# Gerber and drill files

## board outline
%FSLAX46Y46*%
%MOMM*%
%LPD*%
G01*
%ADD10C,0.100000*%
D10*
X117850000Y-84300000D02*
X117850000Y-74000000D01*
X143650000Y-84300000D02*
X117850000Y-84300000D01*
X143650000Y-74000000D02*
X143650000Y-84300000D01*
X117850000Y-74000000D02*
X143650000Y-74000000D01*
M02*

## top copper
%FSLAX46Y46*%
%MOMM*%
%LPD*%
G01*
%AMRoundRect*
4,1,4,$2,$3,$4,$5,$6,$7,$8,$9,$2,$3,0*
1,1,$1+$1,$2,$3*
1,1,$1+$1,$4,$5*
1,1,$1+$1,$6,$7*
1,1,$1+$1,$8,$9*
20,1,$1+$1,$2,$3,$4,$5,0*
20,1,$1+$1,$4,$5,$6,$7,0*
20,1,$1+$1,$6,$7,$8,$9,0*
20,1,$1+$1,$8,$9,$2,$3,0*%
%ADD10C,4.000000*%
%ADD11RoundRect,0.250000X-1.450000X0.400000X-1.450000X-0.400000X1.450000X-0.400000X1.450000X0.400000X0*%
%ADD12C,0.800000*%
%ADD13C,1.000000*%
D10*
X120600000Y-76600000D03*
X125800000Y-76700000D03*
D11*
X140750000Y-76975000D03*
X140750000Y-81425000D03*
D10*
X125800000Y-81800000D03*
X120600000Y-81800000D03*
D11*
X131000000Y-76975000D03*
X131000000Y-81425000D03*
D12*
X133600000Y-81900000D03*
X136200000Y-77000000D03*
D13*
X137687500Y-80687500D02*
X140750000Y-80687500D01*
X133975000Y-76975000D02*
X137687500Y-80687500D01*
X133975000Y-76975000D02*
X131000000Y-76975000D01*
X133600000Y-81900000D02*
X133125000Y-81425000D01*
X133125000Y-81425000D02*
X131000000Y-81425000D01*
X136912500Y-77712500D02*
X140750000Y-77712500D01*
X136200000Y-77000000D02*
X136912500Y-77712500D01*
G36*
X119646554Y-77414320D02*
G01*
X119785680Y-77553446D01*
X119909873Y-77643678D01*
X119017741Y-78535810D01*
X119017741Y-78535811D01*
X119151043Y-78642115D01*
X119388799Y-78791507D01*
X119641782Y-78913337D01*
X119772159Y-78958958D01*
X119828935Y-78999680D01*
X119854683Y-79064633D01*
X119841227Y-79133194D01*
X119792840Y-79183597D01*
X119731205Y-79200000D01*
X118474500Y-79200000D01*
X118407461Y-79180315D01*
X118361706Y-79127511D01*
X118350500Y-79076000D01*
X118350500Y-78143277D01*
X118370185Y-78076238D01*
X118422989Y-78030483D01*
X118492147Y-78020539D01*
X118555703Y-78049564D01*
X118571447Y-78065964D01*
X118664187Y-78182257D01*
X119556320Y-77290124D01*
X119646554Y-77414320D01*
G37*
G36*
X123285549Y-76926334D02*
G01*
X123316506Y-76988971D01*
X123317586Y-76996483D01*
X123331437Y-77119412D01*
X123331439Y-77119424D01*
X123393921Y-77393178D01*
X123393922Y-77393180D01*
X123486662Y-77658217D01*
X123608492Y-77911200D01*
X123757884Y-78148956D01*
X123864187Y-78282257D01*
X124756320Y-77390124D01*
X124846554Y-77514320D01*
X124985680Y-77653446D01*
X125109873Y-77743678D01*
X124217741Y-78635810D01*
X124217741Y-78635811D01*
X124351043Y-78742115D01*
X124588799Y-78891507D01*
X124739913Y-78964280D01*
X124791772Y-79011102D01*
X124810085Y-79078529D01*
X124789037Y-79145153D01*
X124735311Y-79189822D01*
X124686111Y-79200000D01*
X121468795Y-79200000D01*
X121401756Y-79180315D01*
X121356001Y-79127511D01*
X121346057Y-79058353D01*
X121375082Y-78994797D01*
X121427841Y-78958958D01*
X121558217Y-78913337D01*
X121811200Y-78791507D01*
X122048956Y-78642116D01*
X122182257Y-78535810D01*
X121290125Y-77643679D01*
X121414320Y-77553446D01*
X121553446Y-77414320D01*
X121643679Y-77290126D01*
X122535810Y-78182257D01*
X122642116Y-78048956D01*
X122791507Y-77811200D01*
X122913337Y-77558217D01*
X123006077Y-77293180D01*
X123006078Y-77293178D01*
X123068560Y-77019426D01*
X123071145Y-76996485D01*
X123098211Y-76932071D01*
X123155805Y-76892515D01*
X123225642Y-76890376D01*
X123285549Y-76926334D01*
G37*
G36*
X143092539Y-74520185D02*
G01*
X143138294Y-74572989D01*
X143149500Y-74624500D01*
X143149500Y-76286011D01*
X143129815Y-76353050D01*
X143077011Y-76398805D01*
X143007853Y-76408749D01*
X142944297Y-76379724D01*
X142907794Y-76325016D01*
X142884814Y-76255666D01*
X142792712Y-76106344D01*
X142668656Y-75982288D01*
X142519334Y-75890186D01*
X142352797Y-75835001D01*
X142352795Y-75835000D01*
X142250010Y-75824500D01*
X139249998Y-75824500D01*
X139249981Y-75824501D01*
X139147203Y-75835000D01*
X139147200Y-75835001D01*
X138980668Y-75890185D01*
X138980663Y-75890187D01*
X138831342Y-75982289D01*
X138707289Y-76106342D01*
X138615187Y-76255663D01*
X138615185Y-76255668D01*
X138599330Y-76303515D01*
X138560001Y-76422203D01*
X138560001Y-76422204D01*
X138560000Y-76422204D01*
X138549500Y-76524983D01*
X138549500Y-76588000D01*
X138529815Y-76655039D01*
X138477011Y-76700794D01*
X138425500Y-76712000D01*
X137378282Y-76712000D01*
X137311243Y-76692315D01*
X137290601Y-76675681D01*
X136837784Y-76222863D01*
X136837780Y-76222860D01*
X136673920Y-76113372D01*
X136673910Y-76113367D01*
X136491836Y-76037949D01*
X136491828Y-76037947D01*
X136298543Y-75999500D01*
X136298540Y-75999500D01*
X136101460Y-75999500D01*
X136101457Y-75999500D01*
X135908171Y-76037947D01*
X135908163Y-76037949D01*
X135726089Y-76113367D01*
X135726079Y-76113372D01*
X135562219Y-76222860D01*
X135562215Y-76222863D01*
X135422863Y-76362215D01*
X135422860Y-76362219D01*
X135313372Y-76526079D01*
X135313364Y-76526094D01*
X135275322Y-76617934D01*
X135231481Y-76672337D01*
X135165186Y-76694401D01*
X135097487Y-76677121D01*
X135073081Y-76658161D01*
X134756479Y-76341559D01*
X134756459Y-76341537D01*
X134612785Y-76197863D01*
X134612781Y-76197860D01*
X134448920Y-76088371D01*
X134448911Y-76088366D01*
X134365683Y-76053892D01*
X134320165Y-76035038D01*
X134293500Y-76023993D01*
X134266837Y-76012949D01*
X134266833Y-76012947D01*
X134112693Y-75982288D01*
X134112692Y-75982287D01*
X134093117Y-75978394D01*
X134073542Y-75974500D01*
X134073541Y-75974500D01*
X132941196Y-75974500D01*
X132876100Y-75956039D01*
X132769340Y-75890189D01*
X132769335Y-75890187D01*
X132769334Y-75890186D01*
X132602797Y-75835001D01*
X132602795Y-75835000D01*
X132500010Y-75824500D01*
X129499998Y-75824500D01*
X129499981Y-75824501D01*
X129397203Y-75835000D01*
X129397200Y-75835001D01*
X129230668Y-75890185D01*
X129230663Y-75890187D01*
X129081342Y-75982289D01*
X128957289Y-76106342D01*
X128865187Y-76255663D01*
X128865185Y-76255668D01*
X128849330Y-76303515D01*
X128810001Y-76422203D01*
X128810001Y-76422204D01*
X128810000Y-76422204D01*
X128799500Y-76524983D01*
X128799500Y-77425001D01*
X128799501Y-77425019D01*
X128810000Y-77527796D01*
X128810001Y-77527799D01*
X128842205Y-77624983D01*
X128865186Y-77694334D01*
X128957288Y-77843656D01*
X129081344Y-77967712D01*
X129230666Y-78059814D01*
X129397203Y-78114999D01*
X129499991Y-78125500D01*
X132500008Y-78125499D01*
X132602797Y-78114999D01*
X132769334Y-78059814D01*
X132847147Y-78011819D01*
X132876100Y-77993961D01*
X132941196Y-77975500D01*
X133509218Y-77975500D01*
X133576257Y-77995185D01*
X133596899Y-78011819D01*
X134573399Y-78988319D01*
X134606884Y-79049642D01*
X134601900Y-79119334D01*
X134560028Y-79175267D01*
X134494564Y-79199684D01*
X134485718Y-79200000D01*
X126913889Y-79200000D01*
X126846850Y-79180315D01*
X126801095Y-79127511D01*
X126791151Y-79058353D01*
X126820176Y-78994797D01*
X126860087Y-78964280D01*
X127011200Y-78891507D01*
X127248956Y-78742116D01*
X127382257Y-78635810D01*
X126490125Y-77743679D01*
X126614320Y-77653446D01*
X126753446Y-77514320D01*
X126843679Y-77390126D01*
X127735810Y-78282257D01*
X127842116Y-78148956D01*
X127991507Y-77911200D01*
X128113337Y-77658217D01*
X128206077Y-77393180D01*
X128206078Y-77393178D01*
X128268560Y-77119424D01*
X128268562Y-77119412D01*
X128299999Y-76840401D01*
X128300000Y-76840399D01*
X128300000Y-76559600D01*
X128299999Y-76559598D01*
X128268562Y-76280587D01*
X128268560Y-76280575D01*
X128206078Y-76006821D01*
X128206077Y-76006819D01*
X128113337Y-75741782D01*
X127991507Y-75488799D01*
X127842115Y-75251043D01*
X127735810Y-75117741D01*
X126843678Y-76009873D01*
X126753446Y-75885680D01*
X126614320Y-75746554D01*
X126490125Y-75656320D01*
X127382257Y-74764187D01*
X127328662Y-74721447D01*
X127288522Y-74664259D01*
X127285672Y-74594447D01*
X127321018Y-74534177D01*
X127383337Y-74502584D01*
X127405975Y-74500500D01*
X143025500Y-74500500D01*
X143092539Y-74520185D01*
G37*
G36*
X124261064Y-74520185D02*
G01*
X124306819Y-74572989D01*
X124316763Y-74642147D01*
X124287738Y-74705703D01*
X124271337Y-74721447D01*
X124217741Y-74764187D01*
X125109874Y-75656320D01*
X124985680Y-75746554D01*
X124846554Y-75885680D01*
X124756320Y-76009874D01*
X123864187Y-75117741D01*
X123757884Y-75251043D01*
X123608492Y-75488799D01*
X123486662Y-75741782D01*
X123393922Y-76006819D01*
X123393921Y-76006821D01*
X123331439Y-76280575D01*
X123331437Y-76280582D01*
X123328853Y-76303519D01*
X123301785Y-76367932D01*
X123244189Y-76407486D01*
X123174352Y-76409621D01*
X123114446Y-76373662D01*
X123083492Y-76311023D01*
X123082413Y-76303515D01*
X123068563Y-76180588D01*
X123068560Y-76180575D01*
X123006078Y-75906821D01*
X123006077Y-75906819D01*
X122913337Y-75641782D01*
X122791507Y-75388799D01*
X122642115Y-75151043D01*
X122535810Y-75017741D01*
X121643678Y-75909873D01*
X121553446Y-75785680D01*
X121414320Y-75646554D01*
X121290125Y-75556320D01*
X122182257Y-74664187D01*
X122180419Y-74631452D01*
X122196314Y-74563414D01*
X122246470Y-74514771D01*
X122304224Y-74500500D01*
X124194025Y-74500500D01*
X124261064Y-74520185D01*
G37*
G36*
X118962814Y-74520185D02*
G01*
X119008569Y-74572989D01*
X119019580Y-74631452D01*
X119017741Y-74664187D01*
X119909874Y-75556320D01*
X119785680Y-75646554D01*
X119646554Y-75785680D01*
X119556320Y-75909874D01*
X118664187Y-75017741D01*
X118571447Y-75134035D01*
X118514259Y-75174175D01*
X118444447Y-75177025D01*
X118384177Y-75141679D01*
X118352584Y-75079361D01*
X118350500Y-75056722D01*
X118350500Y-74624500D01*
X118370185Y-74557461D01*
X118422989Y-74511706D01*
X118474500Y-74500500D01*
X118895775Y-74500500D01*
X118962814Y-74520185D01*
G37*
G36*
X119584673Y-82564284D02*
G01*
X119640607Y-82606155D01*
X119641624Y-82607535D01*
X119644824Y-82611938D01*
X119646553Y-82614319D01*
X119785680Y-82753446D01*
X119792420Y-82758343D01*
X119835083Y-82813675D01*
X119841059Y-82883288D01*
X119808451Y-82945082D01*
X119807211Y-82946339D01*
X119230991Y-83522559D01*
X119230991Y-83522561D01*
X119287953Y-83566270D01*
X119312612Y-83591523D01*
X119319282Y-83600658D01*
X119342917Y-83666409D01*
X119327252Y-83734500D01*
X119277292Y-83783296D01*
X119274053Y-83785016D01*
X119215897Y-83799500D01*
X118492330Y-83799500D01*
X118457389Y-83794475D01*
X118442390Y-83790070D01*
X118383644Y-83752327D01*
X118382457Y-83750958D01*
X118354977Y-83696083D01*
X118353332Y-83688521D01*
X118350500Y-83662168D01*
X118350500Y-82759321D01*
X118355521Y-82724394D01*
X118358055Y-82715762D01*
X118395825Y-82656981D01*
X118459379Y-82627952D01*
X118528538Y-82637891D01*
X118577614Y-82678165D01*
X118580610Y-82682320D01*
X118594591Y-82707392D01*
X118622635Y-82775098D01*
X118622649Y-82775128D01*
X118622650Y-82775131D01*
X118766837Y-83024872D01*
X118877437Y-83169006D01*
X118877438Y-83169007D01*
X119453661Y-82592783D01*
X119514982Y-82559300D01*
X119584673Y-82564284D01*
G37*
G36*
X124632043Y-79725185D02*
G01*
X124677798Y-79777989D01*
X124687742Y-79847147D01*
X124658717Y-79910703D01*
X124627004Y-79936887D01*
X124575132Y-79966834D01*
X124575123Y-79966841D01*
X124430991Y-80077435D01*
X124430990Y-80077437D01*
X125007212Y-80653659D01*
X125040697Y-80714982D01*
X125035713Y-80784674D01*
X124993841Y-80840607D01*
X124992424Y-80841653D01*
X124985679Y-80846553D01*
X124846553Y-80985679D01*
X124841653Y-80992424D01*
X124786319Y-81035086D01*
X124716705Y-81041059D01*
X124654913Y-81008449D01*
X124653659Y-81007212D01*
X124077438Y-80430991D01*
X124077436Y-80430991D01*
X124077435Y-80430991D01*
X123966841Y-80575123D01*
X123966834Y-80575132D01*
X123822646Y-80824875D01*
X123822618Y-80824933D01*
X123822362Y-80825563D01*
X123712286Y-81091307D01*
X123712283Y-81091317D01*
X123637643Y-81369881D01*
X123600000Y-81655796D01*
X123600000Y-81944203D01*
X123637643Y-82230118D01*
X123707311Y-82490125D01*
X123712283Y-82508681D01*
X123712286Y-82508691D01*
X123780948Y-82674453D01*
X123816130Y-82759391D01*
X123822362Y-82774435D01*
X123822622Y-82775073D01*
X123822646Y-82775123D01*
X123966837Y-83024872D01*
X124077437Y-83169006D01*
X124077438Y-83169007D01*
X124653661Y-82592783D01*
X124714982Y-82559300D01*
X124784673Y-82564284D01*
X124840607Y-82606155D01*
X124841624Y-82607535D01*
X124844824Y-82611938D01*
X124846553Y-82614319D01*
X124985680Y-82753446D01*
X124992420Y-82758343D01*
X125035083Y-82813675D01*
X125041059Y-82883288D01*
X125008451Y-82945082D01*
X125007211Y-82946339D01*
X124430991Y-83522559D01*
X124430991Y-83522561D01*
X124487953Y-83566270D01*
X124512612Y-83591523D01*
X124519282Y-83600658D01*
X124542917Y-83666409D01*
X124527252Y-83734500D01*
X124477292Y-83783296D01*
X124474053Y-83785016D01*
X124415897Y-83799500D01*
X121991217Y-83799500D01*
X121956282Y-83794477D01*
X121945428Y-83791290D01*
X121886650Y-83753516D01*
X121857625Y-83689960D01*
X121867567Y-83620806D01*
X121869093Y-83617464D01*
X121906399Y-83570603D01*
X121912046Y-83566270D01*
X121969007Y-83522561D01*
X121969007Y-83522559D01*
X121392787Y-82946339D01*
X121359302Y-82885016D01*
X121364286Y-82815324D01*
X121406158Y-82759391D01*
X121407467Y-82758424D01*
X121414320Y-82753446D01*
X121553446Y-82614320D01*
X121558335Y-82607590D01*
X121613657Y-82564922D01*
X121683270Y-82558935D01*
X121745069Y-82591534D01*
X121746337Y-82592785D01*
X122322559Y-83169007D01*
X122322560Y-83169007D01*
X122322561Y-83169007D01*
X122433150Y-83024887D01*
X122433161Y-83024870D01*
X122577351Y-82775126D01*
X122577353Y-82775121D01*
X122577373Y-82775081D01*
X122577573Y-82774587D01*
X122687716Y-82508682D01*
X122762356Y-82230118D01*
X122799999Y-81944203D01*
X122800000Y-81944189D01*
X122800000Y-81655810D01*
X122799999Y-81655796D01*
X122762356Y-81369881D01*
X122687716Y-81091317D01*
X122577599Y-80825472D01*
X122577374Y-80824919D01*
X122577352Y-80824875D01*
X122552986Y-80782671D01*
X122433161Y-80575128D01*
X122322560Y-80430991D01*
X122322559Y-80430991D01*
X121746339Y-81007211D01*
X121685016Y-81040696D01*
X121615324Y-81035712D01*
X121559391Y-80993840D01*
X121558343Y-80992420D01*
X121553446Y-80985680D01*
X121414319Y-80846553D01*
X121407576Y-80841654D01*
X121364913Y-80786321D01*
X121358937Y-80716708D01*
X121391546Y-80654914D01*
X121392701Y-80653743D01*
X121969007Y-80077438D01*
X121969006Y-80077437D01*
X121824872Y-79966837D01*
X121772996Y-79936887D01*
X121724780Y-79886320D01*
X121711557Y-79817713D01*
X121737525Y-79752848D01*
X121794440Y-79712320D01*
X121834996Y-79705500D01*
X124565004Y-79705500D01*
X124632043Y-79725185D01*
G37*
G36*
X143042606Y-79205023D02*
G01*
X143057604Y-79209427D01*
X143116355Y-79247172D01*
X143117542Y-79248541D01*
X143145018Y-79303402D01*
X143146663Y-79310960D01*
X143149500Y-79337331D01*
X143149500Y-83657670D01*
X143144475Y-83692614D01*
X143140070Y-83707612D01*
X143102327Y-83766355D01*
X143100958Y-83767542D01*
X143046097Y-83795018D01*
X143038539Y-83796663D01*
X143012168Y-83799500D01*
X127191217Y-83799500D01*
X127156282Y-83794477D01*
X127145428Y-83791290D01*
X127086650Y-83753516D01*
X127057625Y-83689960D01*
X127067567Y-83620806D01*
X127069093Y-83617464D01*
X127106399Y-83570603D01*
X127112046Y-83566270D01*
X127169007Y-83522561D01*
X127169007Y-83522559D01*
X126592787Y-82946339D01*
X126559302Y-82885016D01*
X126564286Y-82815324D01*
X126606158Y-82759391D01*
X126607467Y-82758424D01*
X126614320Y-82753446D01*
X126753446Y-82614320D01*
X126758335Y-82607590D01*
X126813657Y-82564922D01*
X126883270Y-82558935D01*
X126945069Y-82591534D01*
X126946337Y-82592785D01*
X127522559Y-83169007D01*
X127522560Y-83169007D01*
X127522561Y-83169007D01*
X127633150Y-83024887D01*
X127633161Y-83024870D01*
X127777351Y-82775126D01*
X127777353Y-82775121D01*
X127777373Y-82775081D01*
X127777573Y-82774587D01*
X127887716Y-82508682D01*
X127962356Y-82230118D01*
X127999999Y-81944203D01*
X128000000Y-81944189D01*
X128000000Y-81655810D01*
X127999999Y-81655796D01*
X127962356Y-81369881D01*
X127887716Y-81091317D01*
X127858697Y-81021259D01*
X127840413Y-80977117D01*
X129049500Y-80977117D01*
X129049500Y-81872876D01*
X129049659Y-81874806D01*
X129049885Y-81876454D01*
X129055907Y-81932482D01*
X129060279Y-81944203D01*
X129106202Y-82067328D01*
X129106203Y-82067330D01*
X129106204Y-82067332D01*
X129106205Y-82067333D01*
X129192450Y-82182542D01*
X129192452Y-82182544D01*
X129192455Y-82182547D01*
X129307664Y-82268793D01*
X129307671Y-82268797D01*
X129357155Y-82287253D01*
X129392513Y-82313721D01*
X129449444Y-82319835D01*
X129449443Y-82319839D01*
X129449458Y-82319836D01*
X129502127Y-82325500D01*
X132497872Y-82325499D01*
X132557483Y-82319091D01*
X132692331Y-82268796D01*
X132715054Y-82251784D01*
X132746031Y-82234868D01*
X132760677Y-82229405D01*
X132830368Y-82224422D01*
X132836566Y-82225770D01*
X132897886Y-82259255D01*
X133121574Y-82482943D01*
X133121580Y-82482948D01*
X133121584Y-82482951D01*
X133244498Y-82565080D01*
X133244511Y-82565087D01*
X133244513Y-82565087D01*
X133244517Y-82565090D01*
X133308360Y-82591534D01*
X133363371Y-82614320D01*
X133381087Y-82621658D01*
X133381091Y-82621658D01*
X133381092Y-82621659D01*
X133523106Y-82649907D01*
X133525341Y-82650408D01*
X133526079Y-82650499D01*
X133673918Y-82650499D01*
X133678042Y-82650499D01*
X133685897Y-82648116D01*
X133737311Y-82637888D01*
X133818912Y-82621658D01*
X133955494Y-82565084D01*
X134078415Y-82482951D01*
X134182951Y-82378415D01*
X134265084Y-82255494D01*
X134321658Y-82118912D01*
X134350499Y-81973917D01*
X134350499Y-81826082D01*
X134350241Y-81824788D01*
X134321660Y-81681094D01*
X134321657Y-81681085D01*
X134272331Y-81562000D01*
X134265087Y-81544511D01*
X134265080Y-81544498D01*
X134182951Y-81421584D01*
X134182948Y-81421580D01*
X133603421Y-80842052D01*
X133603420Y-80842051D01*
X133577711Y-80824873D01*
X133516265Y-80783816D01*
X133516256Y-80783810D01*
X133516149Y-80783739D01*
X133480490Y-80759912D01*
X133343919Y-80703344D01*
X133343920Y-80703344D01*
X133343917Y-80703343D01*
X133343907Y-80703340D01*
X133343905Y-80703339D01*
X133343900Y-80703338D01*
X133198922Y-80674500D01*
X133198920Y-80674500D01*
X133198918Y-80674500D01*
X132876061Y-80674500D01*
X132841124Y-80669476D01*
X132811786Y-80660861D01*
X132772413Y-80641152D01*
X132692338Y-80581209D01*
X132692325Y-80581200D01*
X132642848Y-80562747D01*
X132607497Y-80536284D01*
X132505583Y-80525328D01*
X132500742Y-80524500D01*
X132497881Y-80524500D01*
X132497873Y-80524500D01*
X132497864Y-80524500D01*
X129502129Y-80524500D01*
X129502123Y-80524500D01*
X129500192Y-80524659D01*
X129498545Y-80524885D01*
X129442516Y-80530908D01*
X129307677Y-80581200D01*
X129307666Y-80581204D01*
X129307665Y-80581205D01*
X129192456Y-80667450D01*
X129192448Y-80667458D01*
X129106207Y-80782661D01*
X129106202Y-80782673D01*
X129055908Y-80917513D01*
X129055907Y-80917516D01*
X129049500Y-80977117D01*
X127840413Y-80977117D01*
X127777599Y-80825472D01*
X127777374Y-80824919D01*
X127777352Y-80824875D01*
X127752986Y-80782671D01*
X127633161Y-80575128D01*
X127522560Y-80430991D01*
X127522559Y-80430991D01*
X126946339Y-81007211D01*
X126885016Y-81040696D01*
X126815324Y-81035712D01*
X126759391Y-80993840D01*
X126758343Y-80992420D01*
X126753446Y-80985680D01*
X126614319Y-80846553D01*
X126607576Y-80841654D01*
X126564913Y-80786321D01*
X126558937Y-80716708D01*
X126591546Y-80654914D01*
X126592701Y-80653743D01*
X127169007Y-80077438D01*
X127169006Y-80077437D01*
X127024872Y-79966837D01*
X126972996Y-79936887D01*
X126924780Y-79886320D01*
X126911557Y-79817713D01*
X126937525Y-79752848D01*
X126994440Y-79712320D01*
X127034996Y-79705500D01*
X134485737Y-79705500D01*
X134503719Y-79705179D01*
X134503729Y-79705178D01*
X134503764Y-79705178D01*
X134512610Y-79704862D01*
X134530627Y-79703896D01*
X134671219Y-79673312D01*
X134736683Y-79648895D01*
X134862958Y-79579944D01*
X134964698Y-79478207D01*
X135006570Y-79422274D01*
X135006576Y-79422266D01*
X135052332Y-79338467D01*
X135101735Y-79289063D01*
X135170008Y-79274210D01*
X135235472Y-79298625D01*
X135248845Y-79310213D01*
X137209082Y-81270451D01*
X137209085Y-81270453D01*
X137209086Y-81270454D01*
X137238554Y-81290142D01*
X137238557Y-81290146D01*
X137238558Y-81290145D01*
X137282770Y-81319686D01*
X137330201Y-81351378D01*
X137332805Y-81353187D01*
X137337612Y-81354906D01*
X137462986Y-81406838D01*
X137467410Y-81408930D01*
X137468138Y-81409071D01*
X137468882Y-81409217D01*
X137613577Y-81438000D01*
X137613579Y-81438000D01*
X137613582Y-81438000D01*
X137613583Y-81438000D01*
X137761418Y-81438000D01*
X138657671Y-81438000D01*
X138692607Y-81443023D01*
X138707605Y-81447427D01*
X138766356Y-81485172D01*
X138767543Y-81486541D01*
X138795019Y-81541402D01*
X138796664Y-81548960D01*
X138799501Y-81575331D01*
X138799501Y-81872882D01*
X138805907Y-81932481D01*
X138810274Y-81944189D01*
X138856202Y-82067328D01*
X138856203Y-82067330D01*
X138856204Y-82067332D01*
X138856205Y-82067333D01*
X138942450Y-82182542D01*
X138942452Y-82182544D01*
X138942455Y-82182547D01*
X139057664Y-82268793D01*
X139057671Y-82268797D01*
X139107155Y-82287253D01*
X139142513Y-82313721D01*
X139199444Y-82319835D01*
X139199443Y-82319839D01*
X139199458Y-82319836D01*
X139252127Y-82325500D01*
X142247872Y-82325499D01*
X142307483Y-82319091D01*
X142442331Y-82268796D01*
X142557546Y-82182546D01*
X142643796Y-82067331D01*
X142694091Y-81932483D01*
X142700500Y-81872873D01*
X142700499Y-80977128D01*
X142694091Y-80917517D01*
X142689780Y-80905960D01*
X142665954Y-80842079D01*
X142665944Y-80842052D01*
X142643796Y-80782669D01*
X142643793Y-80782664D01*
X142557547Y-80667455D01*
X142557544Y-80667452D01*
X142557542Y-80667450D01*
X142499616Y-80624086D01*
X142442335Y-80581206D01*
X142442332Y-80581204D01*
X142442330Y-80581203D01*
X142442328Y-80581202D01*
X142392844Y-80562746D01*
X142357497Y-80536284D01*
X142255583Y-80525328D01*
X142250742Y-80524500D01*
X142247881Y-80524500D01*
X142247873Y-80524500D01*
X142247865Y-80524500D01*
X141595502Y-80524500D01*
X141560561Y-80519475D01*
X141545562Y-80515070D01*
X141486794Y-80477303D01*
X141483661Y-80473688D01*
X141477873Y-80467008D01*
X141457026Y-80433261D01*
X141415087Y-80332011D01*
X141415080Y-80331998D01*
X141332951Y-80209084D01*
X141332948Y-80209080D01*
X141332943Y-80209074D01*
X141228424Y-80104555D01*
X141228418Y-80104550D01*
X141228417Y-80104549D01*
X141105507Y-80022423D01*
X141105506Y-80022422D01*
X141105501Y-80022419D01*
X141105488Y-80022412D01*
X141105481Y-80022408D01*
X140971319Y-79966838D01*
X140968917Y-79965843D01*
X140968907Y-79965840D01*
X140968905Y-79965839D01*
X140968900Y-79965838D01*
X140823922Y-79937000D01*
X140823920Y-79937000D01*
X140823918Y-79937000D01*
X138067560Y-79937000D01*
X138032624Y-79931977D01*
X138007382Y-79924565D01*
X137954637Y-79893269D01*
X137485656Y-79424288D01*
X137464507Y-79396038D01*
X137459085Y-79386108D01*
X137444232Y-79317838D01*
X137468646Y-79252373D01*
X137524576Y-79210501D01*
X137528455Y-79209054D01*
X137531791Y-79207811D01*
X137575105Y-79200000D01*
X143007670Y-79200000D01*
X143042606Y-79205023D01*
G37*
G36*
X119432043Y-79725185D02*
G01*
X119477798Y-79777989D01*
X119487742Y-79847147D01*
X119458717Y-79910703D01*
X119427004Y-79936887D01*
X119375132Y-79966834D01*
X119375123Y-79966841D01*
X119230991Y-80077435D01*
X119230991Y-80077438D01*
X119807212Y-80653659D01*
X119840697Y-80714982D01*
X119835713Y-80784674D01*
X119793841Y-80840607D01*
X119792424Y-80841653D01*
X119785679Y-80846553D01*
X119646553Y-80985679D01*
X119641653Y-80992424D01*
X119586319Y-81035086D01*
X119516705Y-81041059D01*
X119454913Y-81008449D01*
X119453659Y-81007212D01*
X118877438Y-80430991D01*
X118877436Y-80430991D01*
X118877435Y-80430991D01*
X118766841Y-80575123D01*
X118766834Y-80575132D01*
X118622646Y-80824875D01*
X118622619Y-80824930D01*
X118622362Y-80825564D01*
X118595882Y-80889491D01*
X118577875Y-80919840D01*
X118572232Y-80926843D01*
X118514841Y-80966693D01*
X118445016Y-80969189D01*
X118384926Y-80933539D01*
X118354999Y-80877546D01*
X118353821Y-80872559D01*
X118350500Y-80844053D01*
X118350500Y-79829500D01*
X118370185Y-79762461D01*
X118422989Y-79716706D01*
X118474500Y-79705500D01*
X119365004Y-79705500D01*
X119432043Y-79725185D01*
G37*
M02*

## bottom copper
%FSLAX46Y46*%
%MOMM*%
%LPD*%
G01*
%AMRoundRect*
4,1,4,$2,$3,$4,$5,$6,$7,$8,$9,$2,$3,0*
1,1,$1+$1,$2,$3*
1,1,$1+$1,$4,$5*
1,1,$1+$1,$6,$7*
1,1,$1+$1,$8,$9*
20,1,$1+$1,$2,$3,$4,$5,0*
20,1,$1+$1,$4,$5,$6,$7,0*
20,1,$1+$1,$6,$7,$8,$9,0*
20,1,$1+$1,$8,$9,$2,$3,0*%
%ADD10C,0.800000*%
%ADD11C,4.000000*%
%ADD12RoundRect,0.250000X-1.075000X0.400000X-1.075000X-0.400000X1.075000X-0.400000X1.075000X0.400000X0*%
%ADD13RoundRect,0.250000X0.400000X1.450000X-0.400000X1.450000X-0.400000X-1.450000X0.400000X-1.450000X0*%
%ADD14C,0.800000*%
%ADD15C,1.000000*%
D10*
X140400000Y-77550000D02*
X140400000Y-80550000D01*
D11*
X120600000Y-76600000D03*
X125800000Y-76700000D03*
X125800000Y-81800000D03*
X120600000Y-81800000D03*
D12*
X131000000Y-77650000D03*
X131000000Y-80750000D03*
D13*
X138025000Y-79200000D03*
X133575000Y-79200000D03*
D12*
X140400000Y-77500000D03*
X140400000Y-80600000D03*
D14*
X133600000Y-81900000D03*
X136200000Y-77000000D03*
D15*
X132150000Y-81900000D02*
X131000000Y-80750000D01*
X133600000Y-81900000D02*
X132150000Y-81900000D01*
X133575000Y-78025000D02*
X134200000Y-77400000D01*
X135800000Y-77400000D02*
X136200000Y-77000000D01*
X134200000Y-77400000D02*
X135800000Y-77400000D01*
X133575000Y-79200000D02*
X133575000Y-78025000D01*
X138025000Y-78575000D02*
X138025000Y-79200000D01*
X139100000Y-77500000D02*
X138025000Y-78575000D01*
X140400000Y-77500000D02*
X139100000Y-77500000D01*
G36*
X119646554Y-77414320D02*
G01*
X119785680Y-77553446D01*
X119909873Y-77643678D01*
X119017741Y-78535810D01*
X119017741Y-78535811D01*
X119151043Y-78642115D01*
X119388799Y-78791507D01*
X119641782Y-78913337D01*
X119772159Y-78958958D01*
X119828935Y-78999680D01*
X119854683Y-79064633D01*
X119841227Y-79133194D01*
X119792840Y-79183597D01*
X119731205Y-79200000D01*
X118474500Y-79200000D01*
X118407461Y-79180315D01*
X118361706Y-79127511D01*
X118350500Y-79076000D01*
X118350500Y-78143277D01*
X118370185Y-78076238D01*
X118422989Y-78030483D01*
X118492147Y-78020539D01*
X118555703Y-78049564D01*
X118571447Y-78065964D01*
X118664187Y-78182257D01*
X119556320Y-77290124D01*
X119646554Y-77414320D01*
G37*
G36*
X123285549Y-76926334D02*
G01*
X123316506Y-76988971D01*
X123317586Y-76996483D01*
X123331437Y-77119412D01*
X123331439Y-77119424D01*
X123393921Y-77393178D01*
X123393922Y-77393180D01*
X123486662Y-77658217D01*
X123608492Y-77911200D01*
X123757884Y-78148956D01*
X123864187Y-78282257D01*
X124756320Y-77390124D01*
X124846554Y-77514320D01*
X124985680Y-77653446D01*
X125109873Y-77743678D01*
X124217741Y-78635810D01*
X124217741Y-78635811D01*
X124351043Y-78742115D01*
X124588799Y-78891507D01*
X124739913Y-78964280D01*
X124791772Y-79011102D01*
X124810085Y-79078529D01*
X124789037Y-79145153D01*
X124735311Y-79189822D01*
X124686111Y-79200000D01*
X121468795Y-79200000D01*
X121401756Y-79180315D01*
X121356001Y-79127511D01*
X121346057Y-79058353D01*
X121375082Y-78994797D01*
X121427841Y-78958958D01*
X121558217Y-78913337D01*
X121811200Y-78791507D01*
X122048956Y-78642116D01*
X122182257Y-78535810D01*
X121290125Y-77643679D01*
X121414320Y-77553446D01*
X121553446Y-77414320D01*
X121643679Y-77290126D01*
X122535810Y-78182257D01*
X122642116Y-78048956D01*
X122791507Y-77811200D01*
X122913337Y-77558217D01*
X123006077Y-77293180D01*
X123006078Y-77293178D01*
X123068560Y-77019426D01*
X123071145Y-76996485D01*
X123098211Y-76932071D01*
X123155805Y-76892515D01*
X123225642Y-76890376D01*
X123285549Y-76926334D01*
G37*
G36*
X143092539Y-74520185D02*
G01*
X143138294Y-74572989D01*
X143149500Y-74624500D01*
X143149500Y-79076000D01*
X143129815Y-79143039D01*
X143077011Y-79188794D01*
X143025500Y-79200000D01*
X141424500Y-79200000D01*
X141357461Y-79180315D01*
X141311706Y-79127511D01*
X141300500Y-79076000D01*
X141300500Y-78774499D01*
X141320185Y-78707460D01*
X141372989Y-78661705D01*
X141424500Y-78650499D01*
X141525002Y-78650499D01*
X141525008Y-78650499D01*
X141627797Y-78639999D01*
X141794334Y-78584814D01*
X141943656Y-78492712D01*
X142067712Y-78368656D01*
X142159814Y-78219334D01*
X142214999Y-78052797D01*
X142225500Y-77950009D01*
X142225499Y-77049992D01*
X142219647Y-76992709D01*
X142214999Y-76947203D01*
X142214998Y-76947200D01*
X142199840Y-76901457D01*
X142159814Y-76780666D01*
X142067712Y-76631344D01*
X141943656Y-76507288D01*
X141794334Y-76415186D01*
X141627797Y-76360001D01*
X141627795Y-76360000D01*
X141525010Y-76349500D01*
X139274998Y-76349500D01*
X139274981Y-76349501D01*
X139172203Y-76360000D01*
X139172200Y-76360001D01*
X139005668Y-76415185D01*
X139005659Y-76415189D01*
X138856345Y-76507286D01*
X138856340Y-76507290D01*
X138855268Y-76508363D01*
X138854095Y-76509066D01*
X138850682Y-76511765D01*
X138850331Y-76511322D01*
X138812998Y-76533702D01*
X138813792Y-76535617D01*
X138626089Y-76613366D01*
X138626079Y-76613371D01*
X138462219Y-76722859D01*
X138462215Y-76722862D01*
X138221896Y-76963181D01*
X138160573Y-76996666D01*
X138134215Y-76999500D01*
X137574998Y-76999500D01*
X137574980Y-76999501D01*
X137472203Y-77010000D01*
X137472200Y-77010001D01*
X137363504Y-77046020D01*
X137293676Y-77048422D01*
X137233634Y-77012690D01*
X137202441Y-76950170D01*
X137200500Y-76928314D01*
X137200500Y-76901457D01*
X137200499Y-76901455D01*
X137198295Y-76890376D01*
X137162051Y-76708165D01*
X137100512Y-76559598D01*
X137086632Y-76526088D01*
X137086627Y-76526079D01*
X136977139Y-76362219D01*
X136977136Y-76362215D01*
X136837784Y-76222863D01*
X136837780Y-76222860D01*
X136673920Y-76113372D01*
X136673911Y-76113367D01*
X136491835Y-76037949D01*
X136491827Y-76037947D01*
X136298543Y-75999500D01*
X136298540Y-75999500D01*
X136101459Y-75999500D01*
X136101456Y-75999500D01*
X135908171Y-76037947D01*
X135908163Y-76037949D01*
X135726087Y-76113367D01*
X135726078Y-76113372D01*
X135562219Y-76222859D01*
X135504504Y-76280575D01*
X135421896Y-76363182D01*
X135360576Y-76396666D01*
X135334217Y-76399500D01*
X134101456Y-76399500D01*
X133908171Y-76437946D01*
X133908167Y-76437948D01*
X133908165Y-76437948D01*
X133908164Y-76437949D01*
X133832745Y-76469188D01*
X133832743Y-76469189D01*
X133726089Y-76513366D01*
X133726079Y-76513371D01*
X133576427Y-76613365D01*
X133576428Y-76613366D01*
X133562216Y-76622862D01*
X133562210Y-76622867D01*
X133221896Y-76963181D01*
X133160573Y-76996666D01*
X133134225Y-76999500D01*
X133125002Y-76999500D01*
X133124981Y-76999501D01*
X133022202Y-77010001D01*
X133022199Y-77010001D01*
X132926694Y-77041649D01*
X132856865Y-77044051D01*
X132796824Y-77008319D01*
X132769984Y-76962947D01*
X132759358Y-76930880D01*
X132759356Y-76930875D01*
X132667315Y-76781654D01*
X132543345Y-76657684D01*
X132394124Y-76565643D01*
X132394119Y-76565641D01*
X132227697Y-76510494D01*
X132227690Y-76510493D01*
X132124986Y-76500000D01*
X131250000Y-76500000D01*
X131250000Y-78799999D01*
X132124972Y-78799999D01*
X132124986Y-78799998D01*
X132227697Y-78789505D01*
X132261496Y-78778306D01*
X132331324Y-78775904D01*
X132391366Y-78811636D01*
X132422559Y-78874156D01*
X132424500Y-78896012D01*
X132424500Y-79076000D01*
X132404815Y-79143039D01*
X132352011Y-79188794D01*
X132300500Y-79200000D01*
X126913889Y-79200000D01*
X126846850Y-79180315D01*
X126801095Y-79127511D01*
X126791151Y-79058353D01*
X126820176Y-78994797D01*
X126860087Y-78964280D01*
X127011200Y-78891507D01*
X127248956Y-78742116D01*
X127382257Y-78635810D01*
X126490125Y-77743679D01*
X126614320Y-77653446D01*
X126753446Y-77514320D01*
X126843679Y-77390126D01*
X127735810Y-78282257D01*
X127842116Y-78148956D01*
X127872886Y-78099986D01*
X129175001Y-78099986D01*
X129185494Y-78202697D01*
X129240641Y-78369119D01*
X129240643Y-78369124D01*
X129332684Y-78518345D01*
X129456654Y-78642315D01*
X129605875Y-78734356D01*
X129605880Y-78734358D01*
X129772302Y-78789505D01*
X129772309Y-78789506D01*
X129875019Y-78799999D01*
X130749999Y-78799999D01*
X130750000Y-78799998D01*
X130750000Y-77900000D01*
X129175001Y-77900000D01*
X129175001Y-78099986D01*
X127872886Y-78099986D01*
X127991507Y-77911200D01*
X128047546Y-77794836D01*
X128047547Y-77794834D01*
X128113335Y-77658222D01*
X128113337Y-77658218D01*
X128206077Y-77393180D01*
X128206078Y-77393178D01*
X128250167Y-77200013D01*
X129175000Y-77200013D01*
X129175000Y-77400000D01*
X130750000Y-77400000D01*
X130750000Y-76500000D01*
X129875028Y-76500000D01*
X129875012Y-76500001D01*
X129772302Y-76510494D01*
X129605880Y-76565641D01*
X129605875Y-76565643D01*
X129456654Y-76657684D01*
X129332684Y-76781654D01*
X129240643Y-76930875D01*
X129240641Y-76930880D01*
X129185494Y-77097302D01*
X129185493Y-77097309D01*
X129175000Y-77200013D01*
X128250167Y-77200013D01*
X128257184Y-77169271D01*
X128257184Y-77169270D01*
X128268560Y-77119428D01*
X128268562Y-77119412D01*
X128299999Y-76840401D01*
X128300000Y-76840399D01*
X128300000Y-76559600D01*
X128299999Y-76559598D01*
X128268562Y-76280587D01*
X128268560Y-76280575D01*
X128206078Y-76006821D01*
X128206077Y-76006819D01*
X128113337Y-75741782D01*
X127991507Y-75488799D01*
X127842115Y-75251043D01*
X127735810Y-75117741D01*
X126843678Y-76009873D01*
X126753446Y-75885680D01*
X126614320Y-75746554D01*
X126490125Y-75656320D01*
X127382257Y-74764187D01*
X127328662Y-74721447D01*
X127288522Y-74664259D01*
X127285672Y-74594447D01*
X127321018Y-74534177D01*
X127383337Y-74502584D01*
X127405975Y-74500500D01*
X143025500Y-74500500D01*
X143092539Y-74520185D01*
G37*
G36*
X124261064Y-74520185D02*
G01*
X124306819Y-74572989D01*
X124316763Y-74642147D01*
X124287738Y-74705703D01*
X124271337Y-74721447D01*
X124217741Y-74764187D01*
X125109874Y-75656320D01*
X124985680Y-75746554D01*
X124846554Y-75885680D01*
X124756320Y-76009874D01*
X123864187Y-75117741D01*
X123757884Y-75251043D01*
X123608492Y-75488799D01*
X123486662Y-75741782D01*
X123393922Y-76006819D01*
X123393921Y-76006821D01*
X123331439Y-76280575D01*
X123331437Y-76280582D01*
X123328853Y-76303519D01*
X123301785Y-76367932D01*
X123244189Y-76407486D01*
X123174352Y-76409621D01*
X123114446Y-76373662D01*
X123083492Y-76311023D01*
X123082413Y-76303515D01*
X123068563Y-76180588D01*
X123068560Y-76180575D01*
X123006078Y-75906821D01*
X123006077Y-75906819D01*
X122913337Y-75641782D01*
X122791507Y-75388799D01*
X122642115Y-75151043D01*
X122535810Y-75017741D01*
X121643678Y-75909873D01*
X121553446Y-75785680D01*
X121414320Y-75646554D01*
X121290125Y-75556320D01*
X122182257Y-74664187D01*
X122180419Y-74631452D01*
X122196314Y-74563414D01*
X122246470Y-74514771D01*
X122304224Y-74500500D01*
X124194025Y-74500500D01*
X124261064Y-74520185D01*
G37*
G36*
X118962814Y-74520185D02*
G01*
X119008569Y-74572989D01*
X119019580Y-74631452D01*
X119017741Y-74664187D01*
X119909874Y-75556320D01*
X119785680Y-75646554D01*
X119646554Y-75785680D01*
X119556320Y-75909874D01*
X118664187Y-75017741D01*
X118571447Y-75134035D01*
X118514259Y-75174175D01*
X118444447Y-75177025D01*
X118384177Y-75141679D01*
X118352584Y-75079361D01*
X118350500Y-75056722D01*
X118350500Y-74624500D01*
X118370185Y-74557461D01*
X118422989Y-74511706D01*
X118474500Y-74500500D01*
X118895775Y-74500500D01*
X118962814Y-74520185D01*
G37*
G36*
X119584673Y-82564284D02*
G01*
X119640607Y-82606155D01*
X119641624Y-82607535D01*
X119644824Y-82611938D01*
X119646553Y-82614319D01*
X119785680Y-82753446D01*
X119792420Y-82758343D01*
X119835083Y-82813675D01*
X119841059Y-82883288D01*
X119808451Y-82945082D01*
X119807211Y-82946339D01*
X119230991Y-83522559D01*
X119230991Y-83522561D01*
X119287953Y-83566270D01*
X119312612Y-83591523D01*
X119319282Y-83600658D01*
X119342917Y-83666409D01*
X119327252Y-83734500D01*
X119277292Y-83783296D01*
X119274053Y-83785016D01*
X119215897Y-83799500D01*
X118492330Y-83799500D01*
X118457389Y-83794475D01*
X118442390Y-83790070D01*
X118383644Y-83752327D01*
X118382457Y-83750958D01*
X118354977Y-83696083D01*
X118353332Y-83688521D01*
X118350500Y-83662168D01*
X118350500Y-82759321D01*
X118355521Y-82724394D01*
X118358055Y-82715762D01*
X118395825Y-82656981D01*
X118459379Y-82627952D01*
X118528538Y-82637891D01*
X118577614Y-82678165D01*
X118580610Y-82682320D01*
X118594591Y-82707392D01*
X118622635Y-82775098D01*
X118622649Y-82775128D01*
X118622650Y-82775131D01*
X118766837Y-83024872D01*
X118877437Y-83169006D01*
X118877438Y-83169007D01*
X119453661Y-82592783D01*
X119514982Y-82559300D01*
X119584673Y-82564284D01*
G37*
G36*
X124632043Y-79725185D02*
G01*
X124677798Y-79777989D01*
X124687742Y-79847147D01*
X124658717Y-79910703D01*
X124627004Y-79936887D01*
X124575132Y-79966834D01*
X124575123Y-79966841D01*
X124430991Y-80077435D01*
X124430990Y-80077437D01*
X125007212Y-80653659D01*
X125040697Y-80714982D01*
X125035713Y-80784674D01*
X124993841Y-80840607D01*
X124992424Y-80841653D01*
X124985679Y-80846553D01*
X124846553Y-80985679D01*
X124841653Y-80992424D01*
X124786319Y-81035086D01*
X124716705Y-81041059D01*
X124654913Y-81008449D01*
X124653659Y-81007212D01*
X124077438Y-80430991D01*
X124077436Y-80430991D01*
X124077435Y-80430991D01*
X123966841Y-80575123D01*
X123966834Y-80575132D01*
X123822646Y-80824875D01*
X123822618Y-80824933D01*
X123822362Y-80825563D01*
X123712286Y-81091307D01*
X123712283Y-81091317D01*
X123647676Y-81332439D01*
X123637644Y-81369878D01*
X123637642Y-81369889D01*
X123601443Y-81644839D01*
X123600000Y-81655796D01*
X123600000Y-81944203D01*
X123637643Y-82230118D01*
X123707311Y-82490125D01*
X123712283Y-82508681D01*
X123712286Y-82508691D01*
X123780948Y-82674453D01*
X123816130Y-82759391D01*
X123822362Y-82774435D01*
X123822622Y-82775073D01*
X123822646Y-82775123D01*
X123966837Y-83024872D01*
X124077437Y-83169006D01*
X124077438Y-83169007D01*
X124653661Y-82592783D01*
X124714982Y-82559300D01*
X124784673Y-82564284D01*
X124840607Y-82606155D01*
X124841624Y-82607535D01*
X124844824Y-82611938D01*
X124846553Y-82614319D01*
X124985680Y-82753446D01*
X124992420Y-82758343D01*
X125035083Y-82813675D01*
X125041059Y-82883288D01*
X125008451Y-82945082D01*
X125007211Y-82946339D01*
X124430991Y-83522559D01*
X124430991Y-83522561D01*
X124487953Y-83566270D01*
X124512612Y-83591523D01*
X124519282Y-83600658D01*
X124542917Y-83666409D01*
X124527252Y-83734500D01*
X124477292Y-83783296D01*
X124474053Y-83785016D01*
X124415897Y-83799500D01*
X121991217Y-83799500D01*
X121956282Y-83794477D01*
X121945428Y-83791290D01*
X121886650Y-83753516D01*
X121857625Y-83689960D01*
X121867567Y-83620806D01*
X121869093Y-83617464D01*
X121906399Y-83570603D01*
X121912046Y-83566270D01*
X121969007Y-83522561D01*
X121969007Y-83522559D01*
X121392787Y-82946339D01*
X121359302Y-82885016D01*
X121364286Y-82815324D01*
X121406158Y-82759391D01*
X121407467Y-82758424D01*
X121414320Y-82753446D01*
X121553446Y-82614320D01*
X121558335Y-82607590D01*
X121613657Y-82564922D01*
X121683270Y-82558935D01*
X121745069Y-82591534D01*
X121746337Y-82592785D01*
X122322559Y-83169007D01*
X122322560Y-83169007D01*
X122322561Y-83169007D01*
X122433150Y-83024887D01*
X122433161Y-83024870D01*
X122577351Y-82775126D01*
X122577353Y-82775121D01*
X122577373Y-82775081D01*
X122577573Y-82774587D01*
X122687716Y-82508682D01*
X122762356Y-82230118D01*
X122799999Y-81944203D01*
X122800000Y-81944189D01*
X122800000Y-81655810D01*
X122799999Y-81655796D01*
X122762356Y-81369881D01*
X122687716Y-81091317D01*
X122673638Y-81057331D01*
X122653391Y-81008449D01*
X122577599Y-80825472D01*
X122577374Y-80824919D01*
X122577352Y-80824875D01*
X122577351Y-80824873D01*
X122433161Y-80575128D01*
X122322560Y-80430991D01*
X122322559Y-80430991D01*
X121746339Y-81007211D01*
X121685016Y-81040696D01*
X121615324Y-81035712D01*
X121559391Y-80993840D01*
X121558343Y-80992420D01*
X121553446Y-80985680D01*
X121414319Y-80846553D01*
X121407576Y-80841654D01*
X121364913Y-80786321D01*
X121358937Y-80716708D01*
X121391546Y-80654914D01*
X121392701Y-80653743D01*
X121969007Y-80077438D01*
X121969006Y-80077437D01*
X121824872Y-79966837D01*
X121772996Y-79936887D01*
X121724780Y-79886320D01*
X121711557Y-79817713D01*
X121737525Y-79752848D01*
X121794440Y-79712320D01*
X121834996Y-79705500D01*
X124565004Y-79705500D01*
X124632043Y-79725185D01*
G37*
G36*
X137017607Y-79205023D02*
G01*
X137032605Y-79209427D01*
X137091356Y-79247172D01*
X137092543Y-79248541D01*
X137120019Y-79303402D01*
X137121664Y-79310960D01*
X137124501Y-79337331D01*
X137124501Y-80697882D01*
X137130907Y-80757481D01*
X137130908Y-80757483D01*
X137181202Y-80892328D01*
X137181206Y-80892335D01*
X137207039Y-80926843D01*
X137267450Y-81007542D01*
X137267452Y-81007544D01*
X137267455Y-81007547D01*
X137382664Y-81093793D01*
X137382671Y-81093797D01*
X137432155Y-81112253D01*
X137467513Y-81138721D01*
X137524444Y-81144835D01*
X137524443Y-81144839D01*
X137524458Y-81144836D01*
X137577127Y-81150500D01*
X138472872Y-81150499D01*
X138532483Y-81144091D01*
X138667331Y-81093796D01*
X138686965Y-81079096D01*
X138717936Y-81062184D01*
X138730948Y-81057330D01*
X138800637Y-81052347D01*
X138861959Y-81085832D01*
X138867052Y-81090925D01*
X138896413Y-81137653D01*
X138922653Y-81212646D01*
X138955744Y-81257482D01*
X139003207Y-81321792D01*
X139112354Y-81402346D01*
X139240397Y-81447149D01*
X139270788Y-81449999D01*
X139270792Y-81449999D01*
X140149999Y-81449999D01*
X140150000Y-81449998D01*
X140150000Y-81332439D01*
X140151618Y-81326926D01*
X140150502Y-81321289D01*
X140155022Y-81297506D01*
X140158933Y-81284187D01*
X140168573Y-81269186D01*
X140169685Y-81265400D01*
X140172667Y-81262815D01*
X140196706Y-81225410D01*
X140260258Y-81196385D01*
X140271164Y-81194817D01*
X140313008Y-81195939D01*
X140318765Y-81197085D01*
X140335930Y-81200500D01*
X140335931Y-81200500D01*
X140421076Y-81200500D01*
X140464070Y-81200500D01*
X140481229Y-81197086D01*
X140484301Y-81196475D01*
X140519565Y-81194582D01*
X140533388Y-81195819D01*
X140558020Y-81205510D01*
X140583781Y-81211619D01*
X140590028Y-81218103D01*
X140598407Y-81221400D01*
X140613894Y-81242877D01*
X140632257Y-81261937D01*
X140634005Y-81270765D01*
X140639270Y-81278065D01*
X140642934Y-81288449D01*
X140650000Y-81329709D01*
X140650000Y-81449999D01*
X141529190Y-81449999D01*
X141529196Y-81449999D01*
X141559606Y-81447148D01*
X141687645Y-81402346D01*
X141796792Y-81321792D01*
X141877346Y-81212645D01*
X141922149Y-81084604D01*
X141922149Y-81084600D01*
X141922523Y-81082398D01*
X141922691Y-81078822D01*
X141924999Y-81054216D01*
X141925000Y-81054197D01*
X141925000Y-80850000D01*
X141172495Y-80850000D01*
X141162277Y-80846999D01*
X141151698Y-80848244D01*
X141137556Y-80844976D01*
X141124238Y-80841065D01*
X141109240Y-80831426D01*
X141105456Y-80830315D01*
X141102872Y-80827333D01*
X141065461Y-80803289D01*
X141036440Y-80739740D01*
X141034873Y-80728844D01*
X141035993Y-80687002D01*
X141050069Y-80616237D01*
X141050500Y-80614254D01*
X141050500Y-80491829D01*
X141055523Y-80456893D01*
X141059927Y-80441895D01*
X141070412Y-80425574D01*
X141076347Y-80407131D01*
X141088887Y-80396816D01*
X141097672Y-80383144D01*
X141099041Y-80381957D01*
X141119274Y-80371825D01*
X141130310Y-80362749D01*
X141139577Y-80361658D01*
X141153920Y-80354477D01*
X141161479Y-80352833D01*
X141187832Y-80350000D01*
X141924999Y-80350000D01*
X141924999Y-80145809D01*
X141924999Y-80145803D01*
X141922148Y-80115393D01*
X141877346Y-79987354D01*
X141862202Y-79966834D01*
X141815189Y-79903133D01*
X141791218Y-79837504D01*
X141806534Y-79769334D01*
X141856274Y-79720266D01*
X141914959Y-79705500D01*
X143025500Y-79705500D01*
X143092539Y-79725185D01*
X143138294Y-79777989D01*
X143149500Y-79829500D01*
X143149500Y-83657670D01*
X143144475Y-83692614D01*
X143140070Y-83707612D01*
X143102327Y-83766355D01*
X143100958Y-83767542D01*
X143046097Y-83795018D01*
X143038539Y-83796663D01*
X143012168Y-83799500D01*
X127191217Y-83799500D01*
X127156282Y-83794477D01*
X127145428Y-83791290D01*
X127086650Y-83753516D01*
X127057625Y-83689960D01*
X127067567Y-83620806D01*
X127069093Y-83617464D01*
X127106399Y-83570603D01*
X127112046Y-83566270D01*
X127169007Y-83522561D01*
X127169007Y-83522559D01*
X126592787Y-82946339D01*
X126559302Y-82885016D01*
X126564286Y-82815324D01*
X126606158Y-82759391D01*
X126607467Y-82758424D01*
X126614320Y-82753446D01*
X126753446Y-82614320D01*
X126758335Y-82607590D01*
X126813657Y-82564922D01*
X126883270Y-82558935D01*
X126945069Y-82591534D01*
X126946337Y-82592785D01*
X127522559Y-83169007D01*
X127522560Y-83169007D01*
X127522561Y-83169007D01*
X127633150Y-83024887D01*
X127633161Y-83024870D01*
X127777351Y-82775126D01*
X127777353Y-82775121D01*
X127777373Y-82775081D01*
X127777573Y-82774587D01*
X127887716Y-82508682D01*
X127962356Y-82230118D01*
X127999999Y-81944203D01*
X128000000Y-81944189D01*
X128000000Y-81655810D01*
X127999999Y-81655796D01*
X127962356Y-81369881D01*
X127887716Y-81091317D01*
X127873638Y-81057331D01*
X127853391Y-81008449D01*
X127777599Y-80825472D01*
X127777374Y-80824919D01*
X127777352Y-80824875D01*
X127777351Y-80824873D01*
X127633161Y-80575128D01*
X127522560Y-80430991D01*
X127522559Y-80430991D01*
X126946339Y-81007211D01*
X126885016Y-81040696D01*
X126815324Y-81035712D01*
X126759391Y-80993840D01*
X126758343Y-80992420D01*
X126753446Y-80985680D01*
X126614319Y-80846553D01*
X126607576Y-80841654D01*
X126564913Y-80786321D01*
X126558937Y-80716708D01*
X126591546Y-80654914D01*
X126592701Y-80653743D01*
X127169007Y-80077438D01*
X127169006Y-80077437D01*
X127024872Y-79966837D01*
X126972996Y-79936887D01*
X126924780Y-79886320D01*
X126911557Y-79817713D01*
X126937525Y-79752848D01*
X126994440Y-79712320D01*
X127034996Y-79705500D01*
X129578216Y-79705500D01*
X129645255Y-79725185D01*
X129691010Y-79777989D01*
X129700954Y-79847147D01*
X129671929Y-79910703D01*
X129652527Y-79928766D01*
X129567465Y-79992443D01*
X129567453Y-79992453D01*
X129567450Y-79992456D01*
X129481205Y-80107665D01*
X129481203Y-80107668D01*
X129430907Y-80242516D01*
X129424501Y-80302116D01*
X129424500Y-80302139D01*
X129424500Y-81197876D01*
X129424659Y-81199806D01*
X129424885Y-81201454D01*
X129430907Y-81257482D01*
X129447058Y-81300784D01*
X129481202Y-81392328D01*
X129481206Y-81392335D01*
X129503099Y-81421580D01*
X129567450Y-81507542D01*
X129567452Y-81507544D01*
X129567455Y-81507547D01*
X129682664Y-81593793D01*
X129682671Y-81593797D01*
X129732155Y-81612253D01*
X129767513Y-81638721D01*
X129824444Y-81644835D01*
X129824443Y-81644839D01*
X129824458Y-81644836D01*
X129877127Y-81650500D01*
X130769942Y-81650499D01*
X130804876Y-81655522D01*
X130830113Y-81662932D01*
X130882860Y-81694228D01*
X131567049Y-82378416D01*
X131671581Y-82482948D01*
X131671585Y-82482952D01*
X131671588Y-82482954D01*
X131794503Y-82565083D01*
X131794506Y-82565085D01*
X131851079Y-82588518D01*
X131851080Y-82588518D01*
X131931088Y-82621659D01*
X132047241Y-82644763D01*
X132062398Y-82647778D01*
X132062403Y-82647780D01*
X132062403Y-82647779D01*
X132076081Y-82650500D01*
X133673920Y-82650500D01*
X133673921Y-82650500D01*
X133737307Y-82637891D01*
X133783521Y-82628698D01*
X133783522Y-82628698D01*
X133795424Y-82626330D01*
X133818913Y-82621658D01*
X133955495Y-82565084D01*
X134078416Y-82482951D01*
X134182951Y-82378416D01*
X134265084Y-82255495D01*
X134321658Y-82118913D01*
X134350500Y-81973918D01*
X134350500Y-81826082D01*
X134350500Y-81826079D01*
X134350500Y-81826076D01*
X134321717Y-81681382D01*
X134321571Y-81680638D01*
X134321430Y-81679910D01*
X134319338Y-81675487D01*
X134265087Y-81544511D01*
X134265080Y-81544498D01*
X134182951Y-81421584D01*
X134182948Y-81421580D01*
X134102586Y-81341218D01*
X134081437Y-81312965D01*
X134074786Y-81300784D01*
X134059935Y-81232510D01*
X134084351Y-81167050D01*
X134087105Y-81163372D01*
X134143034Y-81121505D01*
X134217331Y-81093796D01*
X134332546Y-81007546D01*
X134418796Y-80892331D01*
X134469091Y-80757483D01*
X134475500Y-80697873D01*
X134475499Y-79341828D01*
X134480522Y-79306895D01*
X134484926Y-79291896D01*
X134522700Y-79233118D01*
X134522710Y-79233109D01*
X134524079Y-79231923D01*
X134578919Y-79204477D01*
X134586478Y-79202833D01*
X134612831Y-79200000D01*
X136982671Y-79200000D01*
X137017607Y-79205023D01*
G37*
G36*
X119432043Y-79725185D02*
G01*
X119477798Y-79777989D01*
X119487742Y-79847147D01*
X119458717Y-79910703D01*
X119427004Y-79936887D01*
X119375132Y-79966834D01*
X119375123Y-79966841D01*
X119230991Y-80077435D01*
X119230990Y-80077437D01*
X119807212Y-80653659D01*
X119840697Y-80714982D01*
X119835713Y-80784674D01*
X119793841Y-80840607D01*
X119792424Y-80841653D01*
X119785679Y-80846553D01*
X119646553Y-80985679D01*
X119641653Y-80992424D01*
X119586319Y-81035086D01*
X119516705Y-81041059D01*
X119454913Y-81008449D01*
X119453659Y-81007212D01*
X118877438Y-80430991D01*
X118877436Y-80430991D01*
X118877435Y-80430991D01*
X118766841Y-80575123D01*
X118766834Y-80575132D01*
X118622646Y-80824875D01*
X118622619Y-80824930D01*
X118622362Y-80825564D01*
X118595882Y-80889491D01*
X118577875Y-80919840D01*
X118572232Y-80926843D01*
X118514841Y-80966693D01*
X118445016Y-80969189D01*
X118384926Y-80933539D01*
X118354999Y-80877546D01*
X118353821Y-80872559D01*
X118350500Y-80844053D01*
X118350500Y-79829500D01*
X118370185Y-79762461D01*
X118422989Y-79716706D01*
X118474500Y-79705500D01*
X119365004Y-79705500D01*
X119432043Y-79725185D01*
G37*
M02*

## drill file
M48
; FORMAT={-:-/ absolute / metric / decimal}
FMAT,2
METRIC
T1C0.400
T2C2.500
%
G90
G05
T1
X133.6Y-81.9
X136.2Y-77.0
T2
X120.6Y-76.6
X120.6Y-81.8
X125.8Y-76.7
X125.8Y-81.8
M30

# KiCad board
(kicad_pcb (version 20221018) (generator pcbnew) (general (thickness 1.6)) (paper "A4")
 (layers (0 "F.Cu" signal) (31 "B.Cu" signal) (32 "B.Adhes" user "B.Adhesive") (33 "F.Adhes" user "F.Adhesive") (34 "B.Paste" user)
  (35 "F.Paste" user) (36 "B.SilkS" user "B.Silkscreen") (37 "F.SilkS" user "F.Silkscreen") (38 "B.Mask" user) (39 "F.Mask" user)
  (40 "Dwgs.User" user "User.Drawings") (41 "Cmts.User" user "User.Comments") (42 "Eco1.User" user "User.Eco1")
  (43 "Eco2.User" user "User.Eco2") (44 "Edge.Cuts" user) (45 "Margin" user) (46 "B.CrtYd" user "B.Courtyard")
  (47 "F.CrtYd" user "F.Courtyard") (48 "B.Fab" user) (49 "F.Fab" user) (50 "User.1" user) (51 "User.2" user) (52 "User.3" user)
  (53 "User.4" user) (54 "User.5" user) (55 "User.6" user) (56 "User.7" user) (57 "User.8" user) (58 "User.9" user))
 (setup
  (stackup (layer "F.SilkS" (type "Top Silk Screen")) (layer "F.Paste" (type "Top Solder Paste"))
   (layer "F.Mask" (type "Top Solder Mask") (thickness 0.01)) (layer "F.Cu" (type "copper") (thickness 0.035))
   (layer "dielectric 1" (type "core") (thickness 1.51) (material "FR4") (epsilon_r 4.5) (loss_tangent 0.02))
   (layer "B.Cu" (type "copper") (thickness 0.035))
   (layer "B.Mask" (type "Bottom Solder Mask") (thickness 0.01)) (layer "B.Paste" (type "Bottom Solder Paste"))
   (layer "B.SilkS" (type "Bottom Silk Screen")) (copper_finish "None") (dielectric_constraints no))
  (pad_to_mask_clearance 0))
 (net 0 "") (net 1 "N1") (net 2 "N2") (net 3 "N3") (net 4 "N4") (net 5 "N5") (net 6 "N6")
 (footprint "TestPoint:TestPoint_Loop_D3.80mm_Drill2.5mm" (layer "F.Cu") (at 120.6 76.6 180)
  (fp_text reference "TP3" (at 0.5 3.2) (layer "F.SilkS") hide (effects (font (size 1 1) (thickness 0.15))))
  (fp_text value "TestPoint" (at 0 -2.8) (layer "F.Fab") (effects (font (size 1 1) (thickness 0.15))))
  (pad "1" thru_hole circle (at 0 0 180) (size 4 4) (drill 2.5) (layers "*.Cu" "*.Mask") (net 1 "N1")))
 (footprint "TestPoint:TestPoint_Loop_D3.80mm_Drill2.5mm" (layer "F.Cu") (at 125.8 76.7)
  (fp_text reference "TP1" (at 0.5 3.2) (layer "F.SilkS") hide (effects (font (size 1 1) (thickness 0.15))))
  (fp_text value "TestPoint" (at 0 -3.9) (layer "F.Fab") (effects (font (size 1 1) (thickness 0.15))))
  (pad "1" thru_hole circle (at 0 0) (size 4 4) (drill 2.5) (layers "*.Cu" "*.Mask") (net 1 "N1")))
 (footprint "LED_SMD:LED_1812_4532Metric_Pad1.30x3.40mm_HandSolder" (layer "F.Cu") (at 140.75 79.2 -90)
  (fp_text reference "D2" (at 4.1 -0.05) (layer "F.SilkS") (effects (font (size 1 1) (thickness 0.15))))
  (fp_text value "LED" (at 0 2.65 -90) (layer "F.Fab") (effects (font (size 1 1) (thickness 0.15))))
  (pad "1" smd roundrect (at -2.225 0 270) (size 1.3 3.4) (layers "F.Cu" "F.Paste" "F.Mask") (roundrect_rratio 0.1923076923) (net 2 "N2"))
  (pad "2" smd roundrect (at 2.225 0 270) (size 1.3 3.4) (layers "F.Cu" "F.Paste" "F.Mask") (roundrect_rratio 0.1923076923) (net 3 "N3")))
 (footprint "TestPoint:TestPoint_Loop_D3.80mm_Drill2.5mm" (layer "F.Cu") (at 125.8 81.8)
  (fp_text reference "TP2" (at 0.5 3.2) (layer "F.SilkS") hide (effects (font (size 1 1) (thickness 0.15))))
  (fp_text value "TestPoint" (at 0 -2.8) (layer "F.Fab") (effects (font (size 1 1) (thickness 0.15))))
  (pad "1" thru_hole circle (at 0 0) (size 4 4) (drill 2.5) (layers "*.Cu" "*.Mask") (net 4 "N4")))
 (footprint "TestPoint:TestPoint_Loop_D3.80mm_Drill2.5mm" (layer "F.Cu") (at 120.6 81.8 180)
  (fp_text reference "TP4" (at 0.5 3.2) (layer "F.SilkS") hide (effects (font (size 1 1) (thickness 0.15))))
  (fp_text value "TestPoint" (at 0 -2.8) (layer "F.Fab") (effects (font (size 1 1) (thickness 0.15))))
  (pad "1" thru_hole circle (at 0 0 180) (size 4 4) (drill 2.5) (layers "*.Cu" "*.Mask") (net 4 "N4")))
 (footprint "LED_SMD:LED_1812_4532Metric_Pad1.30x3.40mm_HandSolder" (layer "F.Cu") (at 131 79.2 -90)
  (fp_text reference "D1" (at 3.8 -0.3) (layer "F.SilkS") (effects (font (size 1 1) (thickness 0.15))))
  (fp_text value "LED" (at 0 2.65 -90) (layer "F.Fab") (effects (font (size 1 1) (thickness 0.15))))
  (pad "1" smd roundrect (at -2.225 0 270) (size 1.3 3.4) (layers "F.Cu" "F.Paste" "F.Mask") (roundrect_rratio 0.1923076923) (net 3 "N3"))
  (pad "2" smd roundrect (at 2.225 0 270) (size 1.3 3.4) (layers "F.Cu" "F.Paste" "F.Mask") (roundrect_rratio 0.1923076923) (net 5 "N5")))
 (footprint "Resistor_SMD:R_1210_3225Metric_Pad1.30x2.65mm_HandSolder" (layer "B.Cu") (at 131 79.2 -90)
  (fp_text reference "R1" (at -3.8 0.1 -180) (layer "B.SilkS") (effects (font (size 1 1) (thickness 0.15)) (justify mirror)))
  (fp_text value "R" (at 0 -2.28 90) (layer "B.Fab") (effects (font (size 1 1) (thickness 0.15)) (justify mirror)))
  (pad "1" smd roundrect (at -1.55 0 270) (size 1.3 2.65) (layers "B.Cu" "B.Paste" "B.Mask") (roundrect_rratio 0.1923076923) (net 1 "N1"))
  (pad "2" smd roundrect (at 1.55 0 270) (size 1.3 2.65) (layers "B.Cu" "B.Paste" "B.Mask") (roundrect_rratio 0.1923076923) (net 5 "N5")))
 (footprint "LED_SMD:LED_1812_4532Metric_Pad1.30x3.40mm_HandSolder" (layer "B.Cu") (at 135.8 79.2 180)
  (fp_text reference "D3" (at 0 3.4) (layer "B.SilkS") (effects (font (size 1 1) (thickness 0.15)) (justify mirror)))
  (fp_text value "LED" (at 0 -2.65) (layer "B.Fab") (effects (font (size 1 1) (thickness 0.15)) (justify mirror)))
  (pad "1" smd roundrect (at -2.225 0 180) (size 1.3 3.4) (layers "B.Cu" "B.Paste" "B.Mask") (roundrect_rratio 0.1923076923) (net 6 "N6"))
  (pad "2" smd roundrect (at 2.225 0 180) (size 1.3 3.4) (layers "B.Cu" "B.Paste" "B.Mask") (roundrect_rratio 0.1923076923) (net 2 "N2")))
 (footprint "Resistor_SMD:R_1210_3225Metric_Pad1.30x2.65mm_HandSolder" (layer "B.Cu") (at 140.4 79.05 -90)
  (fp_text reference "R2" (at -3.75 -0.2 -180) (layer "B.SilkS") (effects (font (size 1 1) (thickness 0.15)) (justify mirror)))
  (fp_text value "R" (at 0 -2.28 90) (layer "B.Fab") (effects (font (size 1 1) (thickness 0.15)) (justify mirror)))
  (pad "1" smd roundrect (at -1.55 0 270) (size 1.3 2.65) (layers "B.Cu" "B.Paste" "B.Mask") (roundrect_rratio 0.1923076923) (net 6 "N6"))
  (pad "2" smd roundrect (at 1.55 0 270) (size 1.3 2.65) (layers "B.Cu" "B.Paste" "B.Mask") (roundrect_rratio 0.1923076923) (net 4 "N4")))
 (gr_line (start 140.4 77.55) (end 140.4 80.55) (stroke (width 0.8) (type default)) (layer "B.Cu"))
 (gr_line (start 117.85 84.3) (end 117.85 74) (stroke (width 0.1) (type default)) (layer "Edge.Cuts"))
 (gr_line (start 143.65 84.3) (end 117.85 84.3) (stroke (width 0.1) (type default)) (layer "Edge.Cuts"))
 (gr_line (start 143.65 74) (end 143.65 84.3) (stroke (width 0.1) (type default)) (layer "Edge.Cuts"))
 (gr_line (start 117.85 74) (end 143.65 74) (stroke (width 0.1) (type default)) (layer "Edge.Cuts"))
 (segment (start 137.6875 80.6875) (end 140.75 80.6875) (width 1) (layer "F.Cu") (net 3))
 (segment (start 133.975 76.975) (end 137.6875 80.6875) (width 1) (layer "F.Cu") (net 3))
 (segment (start 133.975 76.975) (end 131 76.975) (width 1) (layer "F.Cu") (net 3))
 (segment (start 133.6 81.9) (end 133.125 81.425) (width 1) (layer "F.Cu") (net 5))
 (segment (start 133.125 81.425) (end 131 81.425) (width 1) (layer "F.Cu") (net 5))
 (via (at 133.6 81.9) (size 0.8) (drill 0.4) (layers "F.Cu" "B.Cu") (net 5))
 (segment (start 132.15 81.9) (end 131 80.75) (width 1) (layer "B.Cu") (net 5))
 (segment (start 133.6 81.9) (end 132.15 81.9) (width 1) (layer "B.Cu") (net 5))
 (segment (start 136.9125 77.7125) (end 140.75 77.7125) (width 1) (layer "F.Cu") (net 2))
 (segment (start 136.2 77) (end 136.9125 77.7125) (width 1) (layer "F.Cu") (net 2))
 (via (at 136.2 77) (size 0.8) (drill 0.4) (layers "F.Cu" "B.Cu") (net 2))
 (segment (start 133.575 78.025) (end 134.2 77.4) (width 1) (layer "B.Cu") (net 2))
 (segment (start 135.8 77.4) (end 136.2 77) (width 1) (layer "B.Cu") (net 2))
 (segment (start 134.2 77.4) (end 135.8 77.4) (width 1) (layer "B.Cu") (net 2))
 (segment (start 133.575 79.2) (end 133.575 78.025) (width 1) (layer "B.Cu") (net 2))
 (segment (start 138.025 78.575) (end 138.025 79.2) (width 1) (layer "B.Cu") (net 6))
 (segment (start 139.1 77.5) (end 138.025 78.575) (width 1) (layer "B.Cu") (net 6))
 (segment (start 140.4 77.5) (end 139.1 77.5) (width 1) (layer "B.Cu") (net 6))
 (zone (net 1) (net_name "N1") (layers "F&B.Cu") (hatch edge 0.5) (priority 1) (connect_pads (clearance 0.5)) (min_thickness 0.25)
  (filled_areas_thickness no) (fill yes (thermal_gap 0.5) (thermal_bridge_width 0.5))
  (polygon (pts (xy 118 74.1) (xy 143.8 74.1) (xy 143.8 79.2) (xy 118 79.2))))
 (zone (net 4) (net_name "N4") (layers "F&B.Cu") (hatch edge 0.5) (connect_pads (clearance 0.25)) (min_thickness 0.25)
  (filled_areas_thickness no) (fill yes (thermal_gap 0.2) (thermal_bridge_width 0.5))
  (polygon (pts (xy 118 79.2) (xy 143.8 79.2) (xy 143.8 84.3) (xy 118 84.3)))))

